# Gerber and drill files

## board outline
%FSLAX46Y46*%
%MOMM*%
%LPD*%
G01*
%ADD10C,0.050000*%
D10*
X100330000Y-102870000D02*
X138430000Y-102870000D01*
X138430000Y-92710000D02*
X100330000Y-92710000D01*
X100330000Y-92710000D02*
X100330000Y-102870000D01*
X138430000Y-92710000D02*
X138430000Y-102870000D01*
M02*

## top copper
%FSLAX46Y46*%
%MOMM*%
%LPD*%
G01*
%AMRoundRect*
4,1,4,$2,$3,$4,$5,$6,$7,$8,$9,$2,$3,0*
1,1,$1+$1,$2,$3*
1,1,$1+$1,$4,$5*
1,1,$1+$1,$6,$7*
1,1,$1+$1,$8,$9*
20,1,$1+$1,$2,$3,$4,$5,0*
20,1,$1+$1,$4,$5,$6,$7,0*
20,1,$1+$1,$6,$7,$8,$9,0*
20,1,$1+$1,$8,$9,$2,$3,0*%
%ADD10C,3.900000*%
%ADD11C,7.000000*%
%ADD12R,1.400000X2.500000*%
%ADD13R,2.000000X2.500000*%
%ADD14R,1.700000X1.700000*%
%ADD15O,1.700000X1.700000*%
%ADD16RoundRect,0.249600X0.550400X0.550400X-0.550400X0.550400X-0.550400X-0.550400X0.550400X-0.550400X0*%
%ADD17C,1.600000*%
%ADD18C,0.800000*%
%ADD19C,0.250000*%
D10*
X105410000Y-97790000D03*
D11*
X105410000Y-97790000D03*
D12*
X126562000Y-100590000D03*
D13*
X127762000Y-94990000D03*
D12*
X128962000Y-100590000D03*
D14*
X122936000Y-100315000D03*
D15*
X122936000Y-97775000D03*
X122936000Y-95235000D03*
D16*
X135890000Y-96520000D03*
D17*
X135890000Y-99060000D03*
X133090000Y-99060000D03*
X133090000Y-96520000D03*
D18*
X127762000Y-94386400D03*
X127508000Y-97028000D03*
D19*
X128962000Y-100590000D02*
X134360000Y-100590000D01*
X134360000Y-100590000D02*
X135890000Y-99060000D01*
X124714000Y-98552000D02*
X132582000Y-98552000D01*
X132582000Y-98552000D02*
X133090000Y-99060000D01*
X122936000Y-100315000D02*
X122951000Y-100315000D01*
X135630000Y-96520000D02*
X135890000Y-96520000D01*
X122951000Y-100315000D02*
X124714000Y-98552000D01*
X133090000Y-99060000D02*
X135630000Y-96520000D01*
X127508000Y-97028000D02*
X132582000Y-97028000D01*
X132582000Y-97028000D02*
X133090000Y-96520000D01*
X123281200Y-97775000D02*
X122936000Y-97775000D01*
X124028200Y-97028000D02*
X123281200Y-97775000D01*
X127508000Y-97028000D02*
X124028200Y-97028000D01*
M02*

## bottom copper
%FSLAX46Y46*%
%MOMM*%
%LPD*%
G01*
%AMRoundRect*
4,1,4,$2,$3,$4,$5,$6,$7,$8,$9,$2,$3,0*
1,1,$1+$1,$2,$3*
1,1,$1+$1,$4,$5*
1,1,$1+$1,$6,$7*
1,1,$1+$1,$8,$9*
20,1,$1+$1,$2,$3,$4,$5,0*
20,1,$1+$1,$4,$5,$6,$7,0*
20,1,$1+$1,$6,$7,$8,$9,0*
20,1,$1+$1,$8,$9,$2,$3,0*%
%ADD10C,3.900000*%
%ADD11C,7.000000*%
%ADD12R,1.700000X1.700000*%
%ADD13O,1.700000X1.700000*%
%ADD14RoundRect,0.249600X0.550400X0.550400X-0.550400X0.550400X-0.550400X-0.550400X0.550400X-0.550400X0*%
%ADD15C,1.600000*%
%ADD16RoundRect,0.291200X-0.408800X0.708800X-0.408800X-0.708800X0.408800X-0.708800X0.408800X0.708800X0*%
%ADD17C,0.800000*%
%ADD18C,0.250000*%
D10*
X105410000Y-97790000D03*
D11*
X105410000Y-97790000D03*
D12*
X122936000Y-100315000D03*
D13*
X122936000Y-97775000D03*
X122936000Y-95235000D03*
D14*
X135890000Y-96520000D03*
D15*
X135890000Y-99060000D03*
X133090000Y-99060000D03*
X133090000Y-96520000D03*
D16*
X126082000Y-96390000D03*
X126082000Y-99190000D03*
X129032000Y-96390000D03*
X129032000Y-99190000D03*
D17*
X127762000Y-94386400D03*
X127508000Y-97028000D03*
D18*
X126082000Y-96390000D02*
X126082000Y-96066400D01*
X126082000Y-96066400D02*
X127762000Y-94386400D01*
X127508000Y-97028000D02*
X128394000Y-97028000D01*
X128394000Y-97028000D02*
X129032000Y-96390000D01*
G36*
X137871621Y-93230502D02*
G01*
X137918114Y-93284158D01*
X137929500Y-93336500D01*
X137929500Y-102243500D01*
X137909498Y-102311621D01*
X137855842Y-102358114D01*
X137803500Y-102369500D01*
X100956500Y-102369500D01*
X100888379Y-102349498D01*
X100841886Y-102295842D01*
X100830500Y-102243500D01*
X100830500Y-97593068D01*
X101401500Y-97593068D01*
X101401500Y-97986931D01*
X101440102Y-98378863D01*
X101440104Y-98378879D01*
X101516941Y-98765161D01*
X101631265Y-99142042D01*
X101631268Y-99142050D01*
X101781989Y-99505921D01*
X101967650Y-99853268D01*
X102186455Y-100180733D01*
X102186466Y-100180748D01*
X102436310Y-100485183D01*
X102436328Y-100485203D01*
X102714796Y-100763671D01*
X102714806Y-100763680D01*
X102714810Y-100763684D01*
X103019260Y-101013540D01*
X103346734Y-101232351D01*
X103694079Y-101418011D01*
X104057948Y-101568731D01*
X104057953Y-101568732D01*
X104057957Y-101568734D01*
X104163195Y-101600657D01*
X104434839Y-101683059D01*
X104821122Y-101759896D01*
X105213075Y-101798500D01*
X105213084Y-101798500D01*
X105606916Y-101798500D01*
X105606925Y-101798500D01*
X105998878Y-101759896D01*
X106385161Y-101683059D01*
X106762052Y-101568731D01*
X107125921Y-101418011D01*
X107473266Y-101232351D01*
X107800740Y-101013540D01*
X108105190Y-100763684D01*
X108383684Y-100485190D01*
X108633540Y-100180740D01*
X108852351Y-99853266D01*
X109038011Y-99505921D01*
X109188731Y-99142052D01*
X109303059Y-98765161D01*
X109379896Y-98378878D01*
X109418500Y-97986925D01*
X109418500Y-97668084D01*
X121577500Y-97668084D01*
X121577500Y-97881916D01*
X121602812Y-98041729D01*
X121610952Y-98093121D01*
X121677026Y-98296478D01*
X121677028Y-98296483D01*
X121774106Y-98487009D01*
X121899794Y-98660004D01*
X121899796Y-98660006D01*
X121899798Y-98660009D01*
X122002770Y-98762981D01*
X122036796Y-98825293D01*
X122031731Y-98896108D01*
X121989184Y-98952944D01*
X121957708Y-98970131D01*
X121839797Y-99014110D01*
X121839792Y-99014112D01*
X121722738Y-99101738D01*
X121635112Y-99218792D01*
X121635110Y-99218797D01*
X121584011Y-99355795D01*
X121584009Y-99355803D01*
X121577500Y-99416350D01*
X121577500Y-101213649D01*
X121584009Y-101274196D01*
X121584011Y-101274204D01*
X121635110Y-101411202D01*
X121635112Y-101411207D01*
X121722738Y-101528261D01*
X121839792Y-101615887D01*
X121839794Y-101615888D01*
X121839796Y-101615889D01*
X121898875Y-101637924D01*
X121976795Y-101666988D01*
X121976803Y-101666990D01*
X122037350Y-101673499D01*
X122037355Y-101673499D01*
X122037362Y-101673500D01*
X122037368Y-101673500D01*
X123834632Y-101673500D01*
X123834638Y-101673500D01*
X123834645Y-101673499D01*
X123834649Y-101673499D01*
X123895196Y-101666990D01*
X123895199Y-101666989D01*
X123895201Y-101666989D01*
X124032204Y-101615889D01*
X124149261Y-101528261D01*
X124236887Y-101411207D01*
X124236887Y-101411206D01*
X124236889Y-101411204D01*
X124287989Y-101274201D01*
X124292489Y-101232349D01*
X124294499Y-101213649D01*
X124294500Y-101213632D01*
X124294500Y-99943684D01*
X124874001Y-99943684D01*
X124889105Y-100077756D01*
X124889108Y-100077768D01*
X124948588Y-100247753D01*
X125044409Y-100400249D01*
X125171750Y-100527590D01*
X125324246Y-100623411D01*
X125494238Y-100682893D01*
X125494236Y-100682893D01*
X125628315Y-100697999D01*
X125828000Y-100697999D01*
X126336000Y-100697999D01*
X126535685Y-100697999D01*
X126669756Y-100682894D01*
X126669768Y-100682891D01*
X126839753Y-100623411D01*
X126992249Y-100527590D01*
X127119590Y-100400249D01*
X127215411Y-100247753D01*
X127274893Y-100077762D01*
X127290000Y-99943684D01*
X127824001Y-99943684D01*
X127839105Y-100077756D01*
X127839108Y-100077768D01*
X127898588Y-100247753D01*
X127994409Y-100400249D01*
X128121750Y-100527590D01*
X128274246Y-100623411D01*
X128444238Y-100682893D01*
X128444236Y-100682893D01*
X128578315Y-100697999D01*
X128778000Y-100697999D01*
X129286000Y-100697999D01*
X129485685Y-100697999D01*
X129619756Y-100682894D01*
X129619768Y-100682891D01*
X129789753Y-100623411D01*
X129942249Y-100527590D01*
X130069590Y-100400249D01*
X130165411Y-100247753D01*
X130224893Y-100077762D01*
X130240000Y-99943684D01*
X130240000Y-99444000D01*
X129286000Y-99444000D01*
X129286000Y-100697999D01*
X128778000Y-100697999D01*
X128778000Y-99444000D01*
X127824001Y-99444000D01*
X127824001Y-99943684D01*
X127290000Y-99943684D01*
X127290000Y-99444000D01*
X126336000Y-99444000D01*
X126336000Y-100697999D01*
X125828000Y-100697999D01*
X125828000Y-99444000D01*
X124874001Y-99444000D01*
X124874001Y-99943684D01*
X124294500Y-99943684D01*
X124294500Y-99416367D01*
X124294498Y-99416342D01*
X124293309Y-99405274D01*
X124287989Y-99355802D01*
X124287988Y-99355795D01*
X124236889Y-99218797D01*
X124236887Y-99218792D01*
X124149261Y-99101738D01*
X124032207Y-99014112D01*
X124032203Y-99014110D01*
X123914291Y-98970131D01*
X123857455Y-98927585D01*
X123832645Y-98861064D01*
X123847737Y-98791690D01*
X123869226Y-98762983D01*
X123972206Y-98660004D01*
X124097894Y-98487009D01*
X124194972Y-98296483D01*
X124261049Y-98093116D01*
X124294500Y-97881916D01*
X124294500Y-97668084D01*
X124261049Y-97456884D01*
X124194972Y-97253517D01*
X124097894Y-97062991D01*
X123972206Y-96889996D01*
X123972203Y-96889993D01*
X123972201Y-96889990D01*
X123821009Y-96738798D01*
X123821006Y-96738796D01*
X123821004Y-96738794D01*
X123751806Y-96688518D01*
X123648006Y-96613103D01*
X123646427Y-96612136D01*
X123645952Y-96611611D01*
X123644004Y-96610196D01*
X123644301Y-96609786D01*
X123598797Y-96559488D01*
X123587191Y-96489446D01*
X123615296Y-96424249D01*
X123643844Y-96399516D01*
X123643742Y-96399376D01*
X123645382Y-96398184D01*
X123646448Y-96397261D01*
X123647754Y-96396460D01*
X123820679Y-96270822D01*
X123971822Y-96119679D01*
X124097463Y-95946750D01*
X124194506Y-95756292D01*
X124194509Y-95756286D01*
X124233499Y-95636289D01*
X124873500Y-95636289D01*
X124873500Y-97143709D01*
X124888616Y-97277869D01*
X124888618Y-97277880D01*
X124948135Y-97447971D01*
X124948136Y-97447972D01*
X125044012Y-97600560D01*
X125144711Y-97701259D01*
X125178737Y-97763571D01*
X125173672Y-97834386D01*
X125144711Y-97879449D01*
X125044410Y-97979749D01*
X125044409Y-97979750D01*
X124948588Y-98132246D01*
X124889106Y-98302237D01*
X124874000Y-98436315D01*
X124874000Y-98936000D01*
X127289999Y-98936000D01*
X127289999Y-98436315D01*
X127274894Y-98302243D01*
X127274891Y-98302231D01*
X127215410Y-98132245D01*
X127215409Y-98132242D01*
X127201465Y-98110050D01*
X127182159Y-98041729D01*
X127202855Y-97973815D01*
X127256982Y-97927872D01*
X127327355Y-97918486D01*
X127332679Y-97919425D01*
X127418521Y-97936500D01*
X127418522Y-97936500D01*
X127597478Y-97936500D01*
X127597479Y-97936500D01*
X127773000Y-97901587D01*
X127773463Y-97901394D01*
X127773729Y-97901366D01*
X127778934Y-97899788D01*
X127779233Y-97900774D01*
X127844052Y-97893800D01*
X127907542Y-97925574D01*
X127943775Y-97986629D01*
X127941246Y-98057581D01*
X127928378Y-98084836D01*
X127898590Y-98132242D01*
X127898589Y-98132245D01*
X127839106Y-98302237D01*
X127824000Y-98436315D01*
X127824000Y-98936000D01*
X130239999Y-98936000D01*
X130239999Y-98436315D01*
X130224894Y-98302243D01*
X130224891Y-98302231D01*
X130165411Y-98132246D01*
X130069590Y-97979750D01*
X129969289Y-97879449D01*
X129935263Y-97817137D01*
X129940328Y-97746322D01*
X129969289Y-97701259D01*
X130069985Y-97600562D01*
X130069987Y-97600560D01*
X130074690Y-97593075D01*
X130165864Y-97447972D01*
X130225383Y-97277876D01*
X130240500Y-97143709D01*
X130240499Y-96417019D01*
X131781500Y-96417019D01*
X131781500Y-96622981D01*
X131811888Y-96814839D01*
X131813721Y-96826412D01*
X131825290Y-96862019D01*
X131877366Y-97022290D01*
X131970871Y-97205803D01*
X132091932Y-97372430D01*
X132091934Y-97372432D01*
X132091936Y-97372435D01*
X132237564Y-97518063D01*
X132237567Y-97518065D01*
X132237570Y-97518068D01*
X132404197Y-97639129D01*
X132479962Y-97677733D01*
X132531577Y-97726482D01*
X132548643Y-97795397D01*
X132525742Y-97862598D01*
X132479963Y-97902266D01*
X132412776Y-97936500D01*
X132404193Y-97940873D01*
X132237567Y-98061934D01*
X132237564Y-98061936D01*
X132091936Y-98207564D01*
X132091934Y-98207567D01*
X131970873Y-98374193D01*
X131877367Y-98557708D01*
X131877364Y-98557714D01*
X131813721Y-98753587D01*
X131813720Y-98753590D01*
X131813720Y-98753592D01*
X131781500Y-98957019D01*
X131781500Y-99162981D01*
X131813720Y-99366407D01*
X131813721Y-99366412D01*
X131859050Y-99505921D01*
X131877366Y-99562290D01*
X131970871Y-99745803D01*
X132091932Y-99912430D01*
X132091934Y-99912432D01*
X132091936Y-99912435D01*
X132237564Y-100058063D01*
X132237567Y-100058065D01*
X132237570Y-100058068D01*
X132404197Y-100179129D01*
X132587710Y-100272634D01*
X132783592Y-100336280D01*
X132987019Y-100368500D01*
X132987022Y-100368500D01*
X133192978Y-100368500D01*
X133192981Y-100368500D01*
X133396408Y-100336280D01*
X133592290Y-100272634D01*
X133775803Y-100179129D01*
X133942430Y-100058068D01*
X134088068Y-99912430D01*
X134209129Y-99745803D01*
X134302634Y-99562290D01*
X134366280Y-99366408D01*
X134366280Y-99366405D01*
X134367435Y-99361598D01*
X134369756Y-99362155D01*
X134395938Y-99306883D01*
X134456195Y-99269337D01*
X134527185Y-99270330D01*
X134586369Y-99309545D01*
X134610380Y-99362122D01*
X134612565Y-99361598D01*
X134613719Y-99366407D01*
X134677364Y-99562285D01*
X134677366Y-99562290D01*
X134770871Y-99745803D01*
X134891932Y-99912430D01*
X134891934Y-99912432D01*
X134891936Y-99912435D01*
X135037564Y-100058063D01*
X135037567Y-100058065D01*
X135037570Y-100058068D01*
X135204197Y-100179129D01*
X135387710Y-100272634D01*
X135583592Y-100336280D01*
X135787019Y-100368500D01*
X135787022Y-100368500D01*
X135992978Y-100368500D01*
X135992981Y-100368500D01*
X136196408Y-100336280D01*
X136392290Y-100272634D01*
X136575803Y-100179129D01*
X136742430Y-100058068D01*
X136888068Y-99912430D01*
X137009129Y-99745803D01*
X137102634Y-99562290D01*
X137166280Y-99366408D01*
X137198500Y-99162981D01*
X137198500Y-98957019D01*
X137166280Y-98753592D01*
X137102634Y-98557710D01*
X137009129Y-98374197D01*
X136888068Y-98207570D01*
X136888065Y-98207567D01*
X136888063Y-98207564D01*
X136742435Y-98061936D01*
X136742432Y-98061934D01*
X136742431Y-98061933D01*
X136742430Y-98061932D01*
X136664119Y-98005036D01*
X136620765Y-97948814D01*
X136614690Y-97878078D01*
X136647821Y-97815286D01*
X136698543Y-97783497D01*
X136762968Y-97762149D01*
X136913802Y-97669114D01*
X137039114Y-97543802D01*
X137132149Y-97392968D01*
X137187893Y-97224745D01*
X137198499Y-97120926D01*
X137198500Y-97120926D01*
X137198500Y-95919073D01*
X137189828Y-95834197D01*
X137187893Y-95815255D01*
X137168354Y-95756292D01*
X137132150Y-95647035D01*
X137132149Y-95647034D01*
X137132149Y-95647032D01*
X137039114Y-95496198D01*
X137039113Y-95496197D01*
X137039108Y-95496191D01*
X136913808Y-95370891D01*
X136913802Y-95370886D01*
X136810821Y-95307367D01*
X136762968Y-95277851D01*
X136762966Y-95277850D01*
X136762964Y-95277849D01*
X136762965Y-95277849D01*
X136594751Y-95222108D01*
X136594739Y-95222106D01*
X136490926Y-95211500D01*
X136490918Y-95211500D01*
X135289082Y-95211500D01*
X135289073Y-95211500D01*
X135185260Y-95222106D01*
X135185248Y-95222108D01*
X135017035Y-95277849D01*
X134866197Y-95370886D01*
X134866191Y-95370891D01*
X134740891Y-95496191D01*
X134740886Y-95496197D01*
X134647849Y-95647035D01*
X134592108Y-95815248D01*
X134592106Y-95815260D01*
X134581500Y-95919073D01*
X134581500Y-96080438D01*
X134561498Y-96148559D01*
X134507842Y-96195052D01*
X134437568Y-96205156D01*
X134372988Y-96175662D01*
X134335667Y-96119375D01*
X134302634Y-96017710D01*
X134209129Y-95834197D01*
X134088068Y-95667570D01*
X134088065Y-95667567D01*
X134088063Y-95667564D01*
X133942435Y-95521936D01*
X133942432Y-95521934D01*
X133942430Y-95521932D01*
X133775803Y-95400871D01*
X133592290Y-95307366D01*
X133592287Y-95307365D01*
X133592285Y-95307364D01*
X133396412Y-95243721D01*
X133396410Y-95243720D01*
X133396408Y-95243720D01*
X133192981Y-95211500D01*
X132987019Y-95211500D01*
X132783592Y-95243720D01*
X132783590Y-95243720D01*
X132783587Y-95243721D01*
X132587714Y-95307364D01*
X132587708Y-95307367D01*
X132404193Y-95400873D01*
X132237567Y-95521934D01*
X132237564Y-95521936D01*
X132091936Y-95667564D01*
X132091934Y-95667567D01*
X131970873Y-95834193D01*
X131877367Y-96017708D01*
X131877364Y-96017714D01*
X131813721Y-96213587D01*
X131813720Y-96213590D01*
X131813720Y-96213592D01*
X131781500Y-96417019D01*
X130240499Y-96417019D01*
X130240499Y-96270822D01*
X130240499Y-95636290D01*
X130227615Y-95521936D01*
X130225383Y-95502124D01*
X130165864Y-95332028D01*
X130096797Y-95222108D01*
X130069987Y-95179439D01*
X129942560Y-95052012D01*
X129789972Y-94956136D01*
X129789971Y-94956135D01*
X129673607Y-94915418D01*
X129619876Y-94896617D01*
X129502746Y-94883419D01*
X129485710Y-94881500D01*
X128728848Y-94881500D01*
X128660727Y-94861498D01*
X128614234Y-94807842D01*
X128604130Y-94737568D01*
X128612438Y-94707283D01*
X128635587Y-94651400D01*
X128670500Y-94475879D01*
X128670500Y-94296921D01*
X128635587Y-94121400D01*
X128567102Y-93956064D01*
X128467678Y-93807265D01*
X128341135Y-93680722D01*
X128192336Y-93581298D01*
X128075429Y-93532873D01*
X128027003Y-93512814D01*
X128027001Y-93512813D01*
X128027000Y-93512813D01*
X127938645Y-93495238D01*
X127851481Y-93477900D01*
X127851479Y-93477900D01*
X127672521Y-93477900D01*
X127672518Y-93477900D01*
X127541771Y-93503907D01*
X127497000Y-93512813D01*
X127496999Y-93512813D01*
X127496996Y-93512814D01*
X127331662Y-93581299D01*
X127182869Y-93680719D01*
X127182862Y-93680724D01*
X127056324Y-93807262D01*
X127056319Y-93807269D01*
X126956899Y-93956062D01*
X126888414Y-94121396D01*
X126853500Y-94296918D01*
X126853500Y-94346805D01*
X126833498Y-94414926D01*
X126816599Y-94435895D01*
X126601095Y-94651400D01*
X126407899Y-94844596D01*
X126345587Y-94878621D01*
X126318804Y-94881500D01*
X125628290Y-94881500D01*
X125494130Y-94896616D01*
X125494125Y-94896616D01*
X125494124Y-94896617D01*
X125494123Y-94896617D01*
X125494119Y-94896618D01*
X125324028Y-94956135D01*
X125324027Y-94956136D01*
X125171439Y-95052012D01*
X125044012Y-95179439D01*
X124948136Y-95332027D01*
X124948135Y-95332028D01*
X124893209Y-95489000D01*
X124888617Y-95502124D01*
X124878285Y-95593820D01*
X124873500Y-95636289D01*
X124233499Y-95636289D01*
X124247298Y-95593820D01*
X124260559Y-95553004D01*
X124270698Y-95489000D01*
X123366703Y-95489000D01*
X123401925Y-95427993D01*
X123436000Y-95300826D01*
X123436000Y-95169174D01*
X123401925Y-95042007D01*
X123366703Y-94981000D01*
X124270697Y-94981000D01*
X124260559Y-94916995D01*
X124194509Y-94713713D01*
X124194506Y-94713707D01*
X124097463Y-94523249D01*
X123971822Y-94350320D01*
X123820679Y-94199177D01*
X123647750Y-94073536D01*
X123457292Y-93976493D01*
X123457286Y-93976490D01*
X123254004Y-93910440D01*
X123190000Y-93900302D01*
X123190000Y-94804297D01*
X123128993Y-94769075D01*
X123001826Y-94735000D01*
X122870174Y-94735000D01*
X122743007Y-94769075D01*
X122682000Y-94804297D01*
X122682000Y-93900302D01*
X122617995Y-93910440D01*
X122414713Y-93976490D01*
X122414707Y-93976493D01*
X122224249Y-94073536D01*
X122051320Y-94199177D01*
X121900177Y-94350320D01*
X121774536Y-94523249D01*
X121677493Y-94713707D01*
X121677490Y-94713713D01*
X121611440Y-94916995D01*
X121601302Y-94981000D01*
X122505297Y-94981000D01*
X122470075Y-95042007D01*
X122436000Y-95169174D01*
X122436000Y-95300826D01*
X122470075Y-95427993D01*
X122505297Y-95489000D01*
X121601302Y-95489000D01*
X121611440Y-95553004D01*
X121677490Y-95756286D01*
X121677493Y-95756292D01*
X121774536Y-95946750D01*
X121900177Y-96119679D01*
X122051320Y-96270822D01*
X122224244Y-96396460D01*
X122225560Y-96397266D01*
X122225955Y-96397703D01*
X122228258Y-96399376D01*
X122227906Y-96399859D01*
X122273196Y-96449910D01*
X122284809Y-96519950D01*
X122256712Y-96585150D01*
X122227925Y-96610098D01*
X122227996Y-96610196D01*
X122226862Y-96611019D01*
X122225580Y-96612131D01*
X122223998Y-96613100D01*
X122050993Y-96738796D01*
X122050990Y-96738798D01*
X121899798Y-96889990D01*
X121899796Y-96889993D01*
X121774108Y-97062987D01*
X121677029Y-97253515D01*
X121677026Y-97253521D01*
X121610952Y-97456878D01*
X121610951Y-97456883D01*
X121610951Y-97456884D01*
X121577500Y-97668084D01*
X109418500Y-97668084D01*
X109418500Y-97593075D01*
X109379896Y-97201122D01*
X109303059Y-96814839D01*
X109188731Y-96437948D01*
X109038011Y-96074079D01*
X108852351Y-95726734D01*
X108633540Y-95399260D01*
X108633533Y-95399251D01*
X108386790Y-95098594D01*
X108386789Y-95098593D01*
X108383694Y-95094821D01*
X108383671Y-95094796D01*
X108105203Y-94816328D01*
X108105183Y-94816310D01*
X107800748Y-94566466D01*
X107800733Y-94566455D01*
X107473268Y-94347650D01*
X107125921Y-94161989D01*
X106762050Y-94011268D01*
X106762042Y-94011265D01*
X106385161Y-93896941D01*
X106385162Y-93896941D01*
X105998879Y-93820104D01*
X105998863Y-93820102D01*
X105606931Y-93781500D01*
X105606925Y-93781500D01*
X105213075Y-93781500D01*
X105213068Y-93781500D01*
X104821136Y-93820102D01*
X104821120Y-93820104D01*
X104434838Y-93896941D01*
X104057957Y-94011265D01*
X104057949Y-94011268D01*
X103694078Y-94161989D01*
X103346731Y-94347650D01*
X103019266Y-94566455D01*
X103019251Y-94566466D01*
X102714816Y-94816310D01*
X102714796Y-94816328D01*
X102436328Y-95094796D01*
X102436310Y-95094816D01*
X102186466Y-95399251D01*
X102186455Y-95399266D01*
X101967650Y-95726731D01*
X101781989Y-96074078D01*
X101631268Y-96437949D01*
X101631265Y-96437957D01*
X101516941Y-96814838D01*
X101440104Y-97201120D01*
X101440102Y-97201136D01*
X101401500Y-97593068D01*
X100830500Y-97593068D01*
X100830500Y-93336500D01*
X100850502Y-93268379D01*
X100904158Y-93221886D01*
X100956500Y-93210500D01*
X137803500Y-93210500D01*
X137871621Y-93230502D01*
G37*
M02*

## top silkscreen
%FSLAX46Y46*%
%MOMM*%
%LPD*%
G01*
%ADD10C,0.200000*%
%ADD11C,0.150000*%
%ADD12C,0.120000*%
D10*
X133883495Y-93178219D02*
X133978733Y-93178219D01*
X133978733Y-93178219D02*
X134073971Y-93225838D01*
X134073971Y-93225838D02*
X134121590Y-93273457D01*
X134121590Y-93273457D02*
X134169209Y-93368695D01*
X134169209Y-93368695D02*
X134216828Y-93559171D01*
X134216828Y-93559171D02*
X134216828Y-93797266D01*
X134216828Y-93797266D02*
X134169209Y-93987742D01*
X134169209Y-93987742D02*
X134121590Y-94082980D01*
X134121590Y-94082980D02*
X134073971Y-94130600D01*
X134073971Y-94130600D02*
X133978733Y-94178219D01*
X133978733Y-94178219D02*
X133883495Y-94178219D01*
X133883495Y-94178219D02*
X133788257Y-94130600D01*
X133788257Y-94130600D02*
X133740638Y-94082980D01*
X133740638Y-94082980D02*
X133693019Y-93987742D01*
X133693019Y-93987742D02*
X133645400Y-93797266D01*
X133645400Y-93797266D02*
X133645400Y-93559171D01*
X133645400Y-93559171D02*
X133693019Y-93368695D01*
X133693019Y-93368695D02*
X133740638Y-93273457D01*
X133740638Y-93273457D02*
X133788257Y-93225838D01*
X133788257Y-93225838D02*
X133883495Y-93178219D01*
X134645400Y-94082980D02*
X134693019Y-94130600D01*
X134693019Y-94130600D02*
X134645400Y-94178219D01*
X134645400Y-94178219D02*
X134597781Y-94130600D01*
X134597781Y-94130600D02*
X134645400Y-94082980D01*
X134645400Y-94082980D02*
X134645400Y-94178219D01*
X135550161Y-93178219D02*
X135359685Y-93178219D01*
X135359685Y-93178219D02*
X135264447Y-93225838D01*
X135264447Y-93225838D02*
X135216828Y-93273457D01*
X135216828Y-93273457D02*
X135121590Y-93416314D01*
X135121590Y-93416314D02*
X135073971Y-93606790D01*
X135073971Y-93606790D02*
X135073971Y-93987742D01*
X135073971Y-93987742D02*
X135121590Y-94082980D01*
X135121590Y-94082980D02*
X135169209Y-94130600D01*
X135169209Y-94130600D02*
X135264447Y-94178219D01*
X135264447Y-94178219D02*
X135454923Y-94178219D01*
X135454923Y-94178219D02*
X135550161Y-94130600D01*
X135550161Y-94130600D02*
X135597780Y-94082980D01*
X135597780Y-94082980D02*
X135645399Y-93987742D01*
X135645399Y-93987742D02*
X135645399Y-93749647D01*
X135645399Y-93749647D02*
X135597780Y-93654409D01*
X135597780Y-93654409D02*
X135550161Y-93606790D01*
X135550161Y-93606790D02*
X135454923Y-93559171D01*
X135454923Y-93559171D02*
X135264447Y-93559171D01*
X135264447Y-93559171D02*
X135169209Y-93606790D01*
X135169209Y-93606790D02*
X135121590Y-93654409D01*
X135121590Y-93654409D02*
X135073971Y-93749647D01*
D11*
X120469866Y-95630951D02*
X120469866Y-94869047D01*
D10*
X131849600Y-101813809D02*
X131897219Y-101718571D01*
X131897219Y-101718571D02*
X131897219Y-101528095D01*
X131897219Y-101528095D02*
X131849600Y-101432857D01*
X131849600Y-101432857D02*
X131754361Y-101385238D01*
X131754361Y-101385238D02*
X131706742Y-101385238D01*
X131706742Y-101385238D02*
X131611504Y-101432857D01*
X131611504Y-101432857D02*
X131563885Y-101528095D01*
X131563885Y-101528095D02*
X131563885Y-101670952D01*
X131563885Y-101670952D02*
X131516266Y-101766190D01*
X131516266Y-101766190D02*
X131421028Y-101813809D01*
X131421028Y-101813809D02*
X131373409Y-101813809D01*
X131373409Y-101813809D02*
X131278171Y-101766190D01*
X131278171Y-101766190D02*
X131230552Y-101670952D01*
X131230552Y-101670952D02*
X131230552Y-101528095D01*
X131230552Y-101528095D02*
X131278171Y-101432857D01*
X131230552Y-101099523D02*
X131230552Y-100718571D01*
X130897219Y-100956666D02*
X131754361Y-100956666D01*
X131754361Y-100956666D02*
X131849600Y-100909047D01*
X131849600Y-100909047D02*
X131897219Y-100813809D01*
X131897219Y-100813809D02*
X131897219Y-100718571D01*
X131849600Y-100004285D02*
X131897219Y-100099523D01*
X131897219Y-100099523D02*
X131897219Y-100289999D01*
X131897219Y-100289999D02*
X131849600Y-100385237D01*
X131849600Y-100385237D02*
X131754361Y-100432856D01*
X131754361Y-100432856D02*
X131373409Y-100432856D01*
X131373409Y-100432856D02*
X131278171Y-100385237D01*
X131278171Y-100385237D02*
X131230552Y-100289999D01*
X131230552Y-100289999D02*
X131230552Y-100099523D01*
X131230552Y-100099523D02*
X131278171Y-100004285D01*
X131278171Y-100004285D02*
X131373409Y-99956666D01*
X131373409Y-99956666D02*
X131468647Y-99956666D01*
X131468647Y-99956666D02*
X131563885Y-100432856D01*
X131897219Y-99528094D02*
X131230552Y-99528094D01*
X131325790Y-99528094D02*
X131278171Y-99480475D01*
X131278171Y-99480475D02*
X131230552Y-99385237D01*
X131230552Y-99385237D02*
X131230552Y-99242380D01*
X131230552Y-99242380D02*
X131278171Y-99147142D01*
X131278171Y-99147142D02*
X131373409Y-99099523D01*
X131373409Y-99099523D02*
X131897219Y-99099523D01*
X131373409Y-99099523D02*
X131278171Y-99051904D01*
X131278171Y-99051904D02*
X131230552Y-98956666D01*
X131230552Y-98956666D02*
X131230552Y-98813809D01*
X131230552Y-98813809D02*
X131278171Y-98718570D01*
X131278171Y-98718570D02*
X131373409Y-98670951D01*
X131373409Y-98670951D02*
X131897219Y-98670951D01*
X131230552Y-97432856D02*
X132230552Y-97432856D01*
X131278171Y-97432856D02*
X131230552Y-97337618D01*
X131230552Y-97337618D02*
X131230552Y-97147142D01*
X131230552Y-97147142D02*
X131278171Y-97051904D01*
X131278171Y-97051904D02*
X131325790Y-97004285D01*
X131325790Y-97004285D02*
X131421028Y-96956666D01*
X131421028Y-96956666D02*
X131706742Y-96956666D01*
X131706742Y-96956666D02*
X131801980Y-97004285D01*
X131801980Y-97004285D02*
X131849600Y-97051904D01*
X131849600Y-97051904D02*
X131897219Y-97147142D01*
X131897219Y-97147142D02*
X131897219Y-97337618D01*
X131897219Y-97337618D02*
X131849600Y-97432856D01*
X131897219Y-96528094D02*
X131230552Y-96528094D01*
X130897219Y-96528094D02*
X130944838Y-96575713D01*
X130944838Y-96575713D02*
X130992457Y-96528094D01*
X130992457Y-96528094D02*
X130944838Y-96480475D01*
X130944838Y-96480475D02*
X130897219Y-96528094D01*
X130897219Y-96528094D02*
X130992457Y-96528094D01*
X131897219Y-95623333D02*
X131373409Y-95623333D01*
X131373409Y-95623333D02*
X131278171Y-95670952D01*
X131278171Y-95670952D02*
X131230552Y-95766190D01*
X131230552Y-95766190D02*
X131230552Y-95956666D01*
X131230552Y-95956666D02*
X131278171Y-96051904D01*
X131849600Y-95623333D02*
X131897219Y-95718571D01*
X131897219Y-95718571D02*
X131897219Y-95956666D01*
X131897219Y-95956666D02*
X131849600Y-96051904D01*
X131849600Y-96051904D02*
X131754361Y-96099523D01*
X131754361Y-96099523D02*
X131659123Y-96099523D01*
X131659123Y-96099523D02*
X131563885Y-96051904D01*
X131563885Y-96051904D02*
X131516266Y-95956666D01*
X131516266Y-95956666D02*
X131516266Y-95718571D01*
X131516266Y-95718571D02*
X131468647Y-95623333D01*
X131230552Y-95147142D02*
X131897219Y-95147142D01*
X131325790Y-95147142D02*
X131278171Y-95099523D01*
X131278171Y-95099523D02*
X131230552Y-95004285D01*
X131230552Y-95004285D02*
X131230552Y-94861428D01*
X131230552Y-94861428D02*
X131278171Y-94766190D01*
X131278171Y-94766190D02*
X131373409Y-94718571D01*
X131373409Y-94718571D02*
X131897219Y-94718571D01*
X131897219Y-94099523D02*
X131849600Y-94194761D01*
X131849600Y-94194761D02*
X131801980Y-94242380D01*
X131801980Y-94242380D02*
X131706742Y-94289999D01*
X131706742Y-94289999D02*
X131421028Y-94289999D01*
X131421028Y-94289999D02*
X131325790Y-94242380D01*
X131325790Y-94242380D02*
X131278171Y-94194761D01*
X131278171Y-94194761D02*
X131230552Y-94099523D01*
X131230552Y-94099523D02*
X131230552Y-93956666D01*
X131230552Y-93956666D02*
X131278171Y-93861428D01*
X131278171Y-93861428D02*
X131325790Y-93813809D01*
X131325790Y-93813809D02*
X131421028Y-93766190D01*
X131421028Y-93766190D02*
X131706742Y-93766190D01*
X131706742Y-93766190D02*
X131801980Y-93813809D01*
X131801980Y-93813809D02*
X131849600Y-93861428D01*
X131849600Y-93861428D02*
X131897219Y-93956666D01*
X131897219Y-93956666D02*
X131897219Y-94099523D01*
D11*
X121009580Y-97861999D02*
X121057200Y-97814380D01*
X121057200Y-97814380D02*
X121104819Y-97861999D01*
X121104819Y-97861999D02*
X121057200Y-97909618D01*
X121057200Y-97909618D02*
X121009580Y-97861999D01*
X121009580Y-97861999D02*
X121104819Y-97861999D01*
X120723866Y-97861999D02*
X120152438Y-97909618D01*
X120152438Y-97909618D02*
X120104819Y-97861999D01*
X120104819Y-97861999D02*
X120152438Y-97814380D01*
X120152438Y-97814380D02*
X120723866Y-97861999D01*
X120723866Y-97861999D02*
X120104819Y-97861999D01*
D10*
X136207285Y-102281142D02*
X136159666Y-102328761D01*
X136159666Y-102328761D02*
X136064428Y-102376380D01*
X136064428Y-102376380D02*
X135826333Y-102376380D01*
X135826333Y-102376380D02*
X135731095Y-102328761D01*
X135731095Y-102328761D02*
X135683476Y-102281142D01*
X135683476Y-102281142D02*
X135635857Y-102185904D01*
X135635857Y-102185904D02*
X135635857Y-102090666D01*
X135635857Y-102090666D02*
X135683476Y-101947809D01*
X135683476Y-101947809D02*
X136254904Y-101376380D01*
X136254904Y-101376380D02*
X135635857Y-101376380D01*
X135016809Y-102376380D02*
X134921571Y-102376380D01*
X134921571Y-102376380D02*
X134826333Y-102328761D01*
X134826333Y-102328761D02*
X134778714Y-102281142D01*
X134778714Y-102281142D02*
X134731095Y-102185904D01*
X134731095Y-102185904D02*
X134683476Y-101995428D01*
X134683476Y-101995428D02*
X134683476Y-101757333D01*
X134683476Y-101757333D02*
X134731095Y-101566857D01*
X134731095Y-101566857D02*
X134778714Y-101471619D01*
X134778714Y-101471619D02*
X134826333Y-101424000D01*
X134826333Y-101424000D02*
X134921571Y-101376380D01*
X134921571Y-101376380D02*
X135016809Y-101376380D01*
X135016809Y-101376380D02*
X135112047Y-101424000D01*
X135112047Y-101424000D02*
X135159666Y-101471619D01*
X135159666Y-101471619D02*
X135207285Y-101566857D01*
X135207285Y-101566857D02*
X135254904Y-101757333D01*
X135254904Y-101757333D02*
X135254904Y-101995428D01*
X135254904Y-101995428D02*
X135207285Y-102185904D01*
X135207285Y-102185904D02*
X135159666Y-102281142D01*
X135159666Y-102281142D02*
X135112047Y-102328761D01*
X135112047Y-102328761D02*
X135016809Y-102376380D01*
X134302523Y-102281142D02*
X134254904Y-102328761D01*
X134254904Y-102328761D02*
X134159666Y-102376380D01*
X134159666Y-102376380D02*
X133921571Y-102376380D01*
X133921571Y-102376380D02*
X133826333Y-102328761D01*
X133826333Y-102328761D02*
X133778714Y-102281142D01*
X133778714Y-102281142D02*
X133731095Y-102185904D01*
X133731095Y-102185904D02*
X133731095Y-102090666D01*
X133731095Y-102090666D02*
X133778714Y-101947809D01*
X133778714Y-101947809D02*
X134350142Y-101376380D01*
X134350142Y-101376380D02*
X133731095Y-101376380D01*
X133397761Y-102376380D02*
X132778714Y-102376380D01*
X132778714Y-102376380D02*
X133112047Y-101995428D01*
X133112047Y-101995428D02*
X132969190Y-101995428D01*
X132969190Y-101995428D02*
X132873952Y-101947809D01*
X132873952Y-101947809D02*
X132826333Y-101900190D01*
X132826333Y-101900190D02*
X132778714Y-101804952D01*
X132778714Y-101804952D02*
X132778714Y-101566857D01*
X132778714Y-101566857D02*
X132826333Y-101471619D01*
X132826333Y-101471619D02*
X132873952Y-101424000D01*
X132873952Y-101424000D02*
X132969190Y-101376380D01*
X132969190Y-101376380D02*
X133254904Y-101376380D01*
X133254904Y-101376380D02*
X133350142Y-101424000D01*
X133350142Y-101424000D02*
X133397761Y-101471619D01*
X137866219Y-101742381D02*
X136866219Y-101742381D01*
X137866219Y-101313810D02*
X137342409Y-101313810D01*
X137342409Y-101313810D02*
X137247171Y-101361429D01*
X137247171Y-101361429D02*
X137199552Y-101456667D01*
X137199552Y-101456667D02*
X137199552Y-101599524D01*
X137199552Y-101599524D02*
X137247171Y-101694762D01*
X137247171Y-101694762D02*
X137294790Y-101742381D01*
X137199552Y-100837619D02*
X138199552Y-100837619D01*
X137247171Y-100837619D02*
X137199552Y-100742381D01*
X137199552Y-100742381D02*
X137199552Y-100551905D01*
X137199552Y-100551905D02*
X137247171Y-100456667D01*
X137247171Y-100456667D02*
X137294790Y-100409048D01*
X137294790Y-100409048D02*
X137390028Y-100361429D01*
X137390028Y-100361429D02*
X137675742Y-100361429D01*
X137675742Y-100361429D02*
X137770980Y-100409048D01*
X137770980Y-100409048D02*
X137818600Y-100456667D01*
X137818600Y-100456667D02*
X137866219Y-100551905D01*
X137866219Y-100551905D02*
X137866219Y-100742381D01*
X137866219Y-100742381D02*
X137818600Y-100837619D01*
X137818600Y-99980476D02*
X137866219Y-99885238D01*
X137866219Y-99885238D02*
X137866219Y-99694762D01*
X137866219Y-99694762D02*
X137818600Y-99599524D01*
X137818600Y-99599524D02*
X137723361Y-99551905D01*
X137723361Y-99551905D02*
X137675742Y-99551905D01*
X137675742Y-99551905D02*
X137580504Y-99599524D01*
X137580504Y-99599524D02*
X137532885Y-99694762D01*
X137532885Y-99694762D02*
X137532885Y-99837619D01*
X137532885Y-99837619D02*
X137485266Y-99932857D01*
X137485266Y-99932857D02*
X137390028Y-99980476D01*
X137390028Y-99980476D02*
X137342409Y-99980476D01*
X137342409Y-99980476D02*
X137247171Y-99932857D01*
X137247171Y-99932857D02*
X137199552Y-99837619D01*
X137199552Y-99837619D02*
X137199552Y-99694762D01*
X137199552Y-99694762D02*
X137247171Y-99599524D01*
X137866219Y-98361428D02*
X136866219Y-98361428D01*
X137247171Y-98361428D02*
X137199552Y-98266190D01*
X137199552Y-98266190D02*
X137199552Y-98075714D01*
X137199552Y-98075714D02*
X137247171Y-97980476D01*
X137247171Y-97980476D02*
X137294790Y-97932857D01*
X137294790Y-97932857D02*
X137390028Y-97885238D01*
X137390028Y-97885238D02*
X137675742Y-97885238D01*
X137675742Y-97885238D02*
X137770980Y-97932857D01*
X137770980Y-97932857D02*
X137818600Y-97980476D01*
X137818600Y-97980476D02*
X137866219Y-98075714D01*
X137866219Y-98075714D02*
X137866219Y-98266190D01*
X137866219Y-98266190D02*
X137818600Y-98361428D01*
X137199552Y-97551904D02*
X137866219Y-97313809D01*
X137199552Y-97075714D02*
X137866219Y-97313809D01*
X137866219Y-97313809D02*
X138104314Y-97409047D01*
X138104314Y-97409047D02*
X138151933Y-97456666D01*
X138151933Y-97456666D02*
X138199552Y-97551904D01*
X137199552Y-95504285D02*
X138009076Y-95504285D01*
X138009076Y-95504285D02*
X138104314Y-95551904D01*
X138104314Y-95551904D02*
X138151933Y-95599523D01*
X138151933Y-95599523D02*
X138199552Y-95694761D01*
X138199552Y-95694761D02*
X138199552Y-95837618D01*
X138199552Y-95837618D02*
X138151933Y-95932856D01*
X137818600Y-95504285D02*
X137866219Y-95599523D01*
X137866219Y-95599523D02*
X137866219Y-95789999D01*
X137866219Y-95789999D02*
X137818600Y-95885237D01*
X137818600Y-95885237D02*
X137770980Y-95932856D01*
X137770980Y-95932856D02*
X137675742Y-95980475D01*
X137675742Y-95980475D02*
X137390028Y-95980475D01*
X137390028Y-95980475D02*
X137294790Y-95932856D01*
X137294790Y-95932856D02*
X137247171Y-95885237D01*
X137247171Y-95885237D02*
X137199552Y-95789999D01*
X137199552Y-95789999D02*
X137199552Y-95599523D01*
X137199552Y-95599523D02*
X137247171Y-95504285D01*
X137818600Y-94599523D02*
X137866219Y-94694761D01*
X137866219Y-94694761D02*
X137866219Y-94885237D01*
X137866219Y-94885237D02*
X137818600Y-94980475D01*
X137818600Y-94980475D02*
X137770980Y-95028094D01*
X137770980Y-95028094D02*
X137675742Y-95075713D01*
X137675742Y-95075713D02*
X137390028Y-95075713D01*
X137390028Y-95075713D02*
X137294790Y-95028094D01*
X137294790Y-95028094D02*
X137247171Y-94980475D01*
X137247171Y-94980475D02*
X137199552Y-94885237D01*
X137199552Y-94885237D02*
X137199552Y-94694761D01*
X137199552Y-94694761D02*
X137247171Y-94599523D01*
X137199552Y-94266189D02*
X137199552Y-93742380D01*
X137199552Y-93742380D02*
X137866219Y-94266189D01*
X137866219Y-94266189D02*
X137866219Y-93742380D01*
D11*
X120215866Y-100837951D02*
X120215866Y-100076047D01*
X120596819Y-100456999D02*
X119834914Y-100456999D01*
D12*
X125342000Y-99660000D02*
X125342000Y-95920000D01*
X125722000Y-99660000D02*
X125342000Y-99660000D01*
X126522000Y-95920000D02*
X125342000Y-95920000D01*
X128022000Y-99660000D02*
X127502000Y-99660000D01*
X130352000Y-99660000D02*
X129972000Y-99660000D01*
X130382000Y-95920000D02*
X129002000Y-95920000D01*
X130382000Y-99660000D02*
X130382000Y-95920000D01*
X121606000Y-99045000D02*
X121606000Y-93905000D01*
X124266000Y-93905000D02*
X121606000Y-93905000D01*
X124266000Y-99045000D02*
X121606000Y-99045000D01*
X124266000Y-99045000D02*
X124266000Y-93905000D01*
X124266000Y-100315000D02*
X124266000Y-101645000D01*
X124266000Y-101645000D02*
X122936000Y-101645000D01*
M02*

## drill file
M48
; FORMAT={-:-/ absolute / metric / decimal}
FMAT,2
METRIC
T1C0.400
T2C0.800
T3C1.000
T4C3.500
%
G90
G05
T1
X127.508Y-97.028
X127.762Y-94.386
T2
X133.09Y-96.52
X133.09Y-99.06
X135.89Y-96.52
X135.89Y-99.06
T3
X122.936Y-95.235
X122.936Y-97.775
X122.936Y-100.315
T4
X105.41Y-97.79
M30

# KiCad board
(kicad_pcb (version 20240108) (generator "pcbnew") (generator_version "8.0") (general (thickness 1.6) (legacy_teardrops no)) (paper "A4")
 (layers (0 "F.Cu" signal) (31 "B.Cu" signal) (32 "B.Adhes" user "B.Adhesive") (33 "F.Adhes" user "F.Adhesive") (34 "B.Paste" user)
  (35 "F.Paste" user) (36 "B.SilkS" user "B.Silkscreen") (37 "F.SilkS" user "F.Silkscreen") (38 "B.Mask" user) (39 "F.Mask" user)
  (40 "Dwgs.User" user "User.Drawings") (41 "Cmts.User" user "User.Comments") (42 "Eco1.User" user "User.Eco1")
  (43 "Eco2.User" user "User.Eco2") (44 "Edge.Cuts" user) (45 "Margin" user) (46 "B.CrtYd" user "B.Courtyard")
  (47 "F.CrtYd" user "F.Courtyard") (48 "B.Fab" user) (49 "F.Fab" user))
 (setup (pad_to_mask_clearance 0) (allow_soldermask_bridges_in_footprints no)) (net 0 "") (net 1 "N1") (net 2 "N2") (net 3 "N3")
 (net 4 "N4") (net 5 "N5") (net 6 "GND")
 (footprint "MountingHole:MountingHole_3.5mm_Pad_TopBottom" (layer "F.Cu") (at 105.41 97.79)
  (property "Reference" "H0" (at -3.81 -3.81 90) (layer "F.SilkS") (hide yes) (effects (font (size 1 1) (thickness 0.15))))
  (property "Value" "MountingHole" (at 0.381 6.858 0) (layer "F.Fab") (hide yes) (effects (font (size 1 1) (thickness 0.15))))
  (pad "1" thru_hole circle (at 0 0) (size 3.9 3.9) (drill 3.5) (layers "*.Cu" "*.Mask") (remove_unused_layers no))
  (pad "1" connect circle (at 0 0) (size 7 7) (layers "F.Cu" "F.Mask"))
  (pad "1" connect circle (at 0 0) (size 7 7) (layers "B.Cu" "B.Mask")))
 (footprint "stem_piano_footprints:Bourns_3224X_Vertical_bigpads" (layer "F.Cu") (at 127.762 97.79 180)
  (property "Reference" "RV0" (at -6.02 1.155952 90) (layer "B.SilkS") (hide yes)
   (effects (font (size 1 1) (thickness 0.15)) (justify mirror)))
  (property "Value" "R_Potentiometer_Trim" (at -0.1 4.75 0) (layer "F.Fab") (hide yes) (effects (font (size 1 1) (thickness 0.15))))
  (fp_line (start 2.42 -1.87) (end 2.42 1.87) (stroke (width 0.12) (type solid)) (layer "F.SilkS"))
  (fp_line (start 2.04 -1.87) (end 2.42 -1.87) (stroke (width 0.12) (type solid)) (layer "F.SilkS"))
  (fp_line (start 1.24 1.87) (end 2.42 1.87) (stroke (width 0.12) (type solid)) (layer "F.SilkS"))
  (fp_line (start -0.26 -1.87) (end 0.26 -1.87) (stroke (width 0.12) (type solid)) (layer "F.SilkS"))
  (fp_line (start -2.59 -1.87) (end -2.21 -1.87) (stroke (width 0.12) (type solid)) (layer "F.SilkS"))
  (fp_line (start -2.62 1.87) (end -1.24 1.87) (stroke (width 0.12) (type solid)) (layer "F.SilkS"))
  (fp_line (start -2.62 -1.87) (end -2.62 1.87) (stroke (width 0.12) (type solid)) (layer "F.SilkS"))
  (pad "1" smd rect (at 1.2 -2.8 180) (size 1.4 2.5) (layers "F.Cu" "F.Paste" "F.Mask") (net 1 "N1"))
  (pad "2" smd rect (at 0 2.8 180) (size 2 2.5) (layers "F.Cu" "F.Paste" "F.Mask") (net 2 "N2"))
  (pad "3" smd rect (at -1.2 -2.8 180) (size 1.4 2.5) (layers "F.Cu" "F.Paste" "F.Mask") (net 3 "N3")))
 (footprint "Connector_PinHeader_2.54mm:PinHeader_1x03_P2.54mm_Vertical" (layer "F.Cu") (at 122.936 100.315 180)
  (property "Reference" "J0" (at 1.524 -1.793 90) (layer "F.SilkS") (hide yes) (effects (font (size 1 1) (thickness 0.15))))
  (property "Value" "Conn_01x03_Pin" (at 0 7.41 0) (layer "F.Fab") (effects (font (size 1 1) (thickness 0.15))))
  (fp_line (start 1.33 1.27) (end 1.33 6.41) (stroke (width 0.12) (type solid)) (layer "F.SilkS"))
  (fp_line (start -1.33 6.41) (end 1.33 6.41) (stroke (width 0.12) (type solid)) (layer "F.SilkS"))
  (fp_line (start -1.33 1.27) (end 1.33 1.27) (stroke (width 0.12) (type solid)) (layer "F.SilkS"))
  (fp_line (start -1.33 1.27) (end -1.33 6.41) (stroke (width 0.12) (type solid)) (layer "F.SilkS"))
  (fp_line (start -1.33 0) (end -1.33 -1.33) (stroke (width 0.12) (type solid)) (layer "F.SilkS"))
  (fp_line (start -1.33 -1.33) (end 0 -1.33) (stroke (width 0.12) (type solid)) (layer "F.SilkS"))
  (pad "1" thru_hole rect (at 0 0 180) (size 1.7 1.7) (drill 1) (layers "*.Cu" "*.Mask") (remove_unused_layers no) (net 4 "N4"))
  (pad "2" thru_hole oval (at 0 2.54 180) (size 1.7 1.7) (drill 1) (layers "*.Cu" "*.Mask") (remove_unused_layers no) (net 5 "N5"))
  (pad "3" thru_hole oval (at 0 5.08 180) (size 1.7 1.7) (drill 1) (layers "*.Cu" "*.Mask") (remove_unused_layers no) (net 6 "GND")))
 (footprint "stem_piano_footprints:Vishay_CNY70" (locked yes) (layer "B.Cu") (at 135.89 96.52 180)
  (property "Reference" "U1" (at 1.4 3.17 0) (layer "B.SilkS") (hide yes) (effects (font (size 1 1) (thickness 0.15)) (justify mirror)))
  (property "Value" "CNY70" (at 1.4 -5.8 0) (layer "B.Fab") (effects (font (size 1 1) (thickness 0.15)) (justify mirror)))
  (pad "1" thru_hole roundrect (at 0 0 180) (size 1.6 1.6) (drill 0.8) (layers "*.Cu" "*.Mask") (remove_unused_layers no)
   (roundrect_rratio 0.156) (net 4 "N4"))
  (pad "2" thru_hole circle (at 0 -2.54 180) (size 1.6 1.6) (drill 0.8) (layers "*.Cu" "*.Mask") (remove_unused_layers no) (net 3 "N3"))
  (pad "3" thru_hole circle (at 2.8 -2.54 180) (size 1.6 1.6) (drill 0.8) (layers "*.Cu" "*.Mask") (remove_unused_layers no) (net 4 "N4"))
  (pad "4" thru_hole circle (at 2.8 0 180) (size 1.6 1.6) (drill 0.8) (layers "*.Cu" "*.Mask") (remove_unused_layers no) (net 5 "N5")))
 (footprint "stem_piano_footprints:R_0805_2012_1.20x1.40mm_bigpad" (layer "B.Cu") (at 126.082 97.79 -90)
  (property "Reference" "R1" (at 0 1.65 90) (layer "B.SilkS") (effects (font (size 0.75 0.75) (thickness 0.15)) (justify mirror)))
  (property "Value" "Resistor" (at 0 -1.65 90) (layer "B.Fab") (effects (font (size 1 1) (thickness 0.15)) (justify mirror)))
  (pad "1" smd roundrect (at -1.4 0 270) (size 2 1.4) (layers "B.Cu" "B.Paste" "B.Mask") (roundrect_rratio 0.208) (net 2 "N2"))
  (pad "2" smd roundrect (at 1.4 0 270) (size 2 1.4) (layers "B.Cu" "B.Paste" "B.Mask") (roundrect_rratio 0.208) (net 6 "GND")))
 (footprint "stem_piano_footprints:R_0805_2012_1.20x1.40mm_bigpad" (layer "B.Cu") (at 129.032 97.79 -90)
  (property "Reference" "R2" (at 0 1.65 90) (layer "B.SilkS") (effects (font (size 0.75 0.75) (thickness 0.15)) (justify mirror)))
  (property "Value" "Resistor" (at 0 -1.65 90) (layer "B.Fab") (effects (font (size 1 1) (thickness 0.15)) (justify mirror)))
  (pad "1" smd roundrect (at -1.4 0 270) (size 2 1.4) (layers "B.Cu" "B.Paste" "B.Mask") (roundrect_rratio 0.208) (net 5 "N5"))
  (pad "2" smd roundrect (at 1.4 0 270) (size 2 1.4) (layers "B.Cu" "B.Paste" "B.Mask") (roundrect_rratio 0.208) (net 6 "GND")))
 (gr_line (start 100.33 102.87) (end 138.43 102.87) (stroke (width 0.05) (type solid)) (layer "Edge.Cuts"))
 (gr_line (start 138.43 92.71) (end 100.33 92.71) (stroke (width 0.05) (type solid)) (layer "Edge.Cuts"))
 (gr_line (start 100.33 92.71) (end 100.33 102.87) (stroke (width 0.05) (type solid)) (layer "Edge.Cuts"))
 (gr_line (start 138.43 92.71) (end 138.43 102.87) (stroke (width 0.05) (type solid)) (layer "Edge.Cuts"))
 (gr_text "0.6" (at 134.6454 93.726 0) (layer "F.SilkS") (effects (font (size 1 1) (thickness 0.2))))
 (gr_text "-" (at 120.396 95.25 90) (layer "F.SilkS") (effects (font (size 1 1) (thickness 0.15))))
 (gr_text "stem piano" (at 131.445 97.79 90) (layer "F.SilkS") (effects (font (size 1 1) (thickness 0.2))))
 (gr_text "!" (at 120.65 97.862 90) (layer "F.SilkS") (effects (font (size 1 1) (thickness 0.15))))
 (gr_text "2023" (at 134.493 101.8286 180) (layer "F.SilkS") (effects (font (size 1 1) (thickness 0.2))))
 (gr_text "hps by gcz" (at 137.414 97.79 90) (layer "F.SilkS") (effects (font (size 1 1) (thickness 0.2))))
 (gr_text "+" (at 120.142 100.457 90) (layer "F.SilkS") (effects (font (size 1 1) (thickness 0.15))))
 (via (at 127.762 94.3864) (size 0.8) (drill 0.4) (layers "F.Cu" "B.Cu") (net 2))
 (segment (start 126.082 96.39) (end 126.082 96.0664) (width 0.25) (layer "B.Cu") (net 2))
 (segment (start 126.082 96.0664) (end 127.762 94.3864) (width 0.25) (layer "B.Cu") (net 2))
 (segment (start 128.962 100.59) (end 134.36 100.59) (width 0.25) (layer "F.Cu") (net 3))
 (segment (start 134.36 100.59) (end 135.89 99.06) (width 0.25) (layer "F.Cu") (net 3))
 (segment (start 124.714 98.552) (end 132.582 98.552) (width 0.25) (layer "F.Cu") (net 4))
 (segment (start 132.582 98.552) (end 133.09 99.06) (width 0.25) (layer "F.Cu") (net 4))
 (segment (start 122.936 100.315) (end 122.951 100.315) (width 0.25) (layer "F.Cu") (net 4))
 (segment (start 135.63 96.52) (end 135.89 96.52) (width 0.25) (layer "F.Cu") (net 4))
 (segment (start 122.951 100.315) (end 124.714 98.552) (width 0.25) (layer "F.Cu") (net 4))
 (segment (start 133.09 99.06) (end 135.63 96.52) (width 0.25) (layer "F.Cu") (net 4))
 (segment (start 127.508 97.028) (end 132.582 97.028) (width 0.25) (layer "F.Cu") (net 5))
 (segment (start 132.582 97.028) (end 133.09 96.52) (width 0.25) (layer "F.Cu") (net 5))
 (segment (start 123.2812 97.775) (end 122.936 97.775) (width 0.25) (layer "F.Cu") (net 5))
 (segment (start 124.0282 97.028) (end 123.2812 97.775) (width 0.25) (layer "F.Cu") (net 5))
 (segment (start 127.508 97.028) (end 124.0282 97.028) (width 0.25) (layer "F.Cu") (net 5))
 (via (at 127.508 97.028) (size 0.8) (drill 0.4) (layers "F.Cu" "B.Cu") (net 5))
 (segment (start 127.508 97.028) (end 128.394 97.028) (width 0.25) (layer "B.Cu") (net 5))
 (segment (start 128.394 97.028) (end 129.032 96.39) (width 0.25) (layer "B.Cu") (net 5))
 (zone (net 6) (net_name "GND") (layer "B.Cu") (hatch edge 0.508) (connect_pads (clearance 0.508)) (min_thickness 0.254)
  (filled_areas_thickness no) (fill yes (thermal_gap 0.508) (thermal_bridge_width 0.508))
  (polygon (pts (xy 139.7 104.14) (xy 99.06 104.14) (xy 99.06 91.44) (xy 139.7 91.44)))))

